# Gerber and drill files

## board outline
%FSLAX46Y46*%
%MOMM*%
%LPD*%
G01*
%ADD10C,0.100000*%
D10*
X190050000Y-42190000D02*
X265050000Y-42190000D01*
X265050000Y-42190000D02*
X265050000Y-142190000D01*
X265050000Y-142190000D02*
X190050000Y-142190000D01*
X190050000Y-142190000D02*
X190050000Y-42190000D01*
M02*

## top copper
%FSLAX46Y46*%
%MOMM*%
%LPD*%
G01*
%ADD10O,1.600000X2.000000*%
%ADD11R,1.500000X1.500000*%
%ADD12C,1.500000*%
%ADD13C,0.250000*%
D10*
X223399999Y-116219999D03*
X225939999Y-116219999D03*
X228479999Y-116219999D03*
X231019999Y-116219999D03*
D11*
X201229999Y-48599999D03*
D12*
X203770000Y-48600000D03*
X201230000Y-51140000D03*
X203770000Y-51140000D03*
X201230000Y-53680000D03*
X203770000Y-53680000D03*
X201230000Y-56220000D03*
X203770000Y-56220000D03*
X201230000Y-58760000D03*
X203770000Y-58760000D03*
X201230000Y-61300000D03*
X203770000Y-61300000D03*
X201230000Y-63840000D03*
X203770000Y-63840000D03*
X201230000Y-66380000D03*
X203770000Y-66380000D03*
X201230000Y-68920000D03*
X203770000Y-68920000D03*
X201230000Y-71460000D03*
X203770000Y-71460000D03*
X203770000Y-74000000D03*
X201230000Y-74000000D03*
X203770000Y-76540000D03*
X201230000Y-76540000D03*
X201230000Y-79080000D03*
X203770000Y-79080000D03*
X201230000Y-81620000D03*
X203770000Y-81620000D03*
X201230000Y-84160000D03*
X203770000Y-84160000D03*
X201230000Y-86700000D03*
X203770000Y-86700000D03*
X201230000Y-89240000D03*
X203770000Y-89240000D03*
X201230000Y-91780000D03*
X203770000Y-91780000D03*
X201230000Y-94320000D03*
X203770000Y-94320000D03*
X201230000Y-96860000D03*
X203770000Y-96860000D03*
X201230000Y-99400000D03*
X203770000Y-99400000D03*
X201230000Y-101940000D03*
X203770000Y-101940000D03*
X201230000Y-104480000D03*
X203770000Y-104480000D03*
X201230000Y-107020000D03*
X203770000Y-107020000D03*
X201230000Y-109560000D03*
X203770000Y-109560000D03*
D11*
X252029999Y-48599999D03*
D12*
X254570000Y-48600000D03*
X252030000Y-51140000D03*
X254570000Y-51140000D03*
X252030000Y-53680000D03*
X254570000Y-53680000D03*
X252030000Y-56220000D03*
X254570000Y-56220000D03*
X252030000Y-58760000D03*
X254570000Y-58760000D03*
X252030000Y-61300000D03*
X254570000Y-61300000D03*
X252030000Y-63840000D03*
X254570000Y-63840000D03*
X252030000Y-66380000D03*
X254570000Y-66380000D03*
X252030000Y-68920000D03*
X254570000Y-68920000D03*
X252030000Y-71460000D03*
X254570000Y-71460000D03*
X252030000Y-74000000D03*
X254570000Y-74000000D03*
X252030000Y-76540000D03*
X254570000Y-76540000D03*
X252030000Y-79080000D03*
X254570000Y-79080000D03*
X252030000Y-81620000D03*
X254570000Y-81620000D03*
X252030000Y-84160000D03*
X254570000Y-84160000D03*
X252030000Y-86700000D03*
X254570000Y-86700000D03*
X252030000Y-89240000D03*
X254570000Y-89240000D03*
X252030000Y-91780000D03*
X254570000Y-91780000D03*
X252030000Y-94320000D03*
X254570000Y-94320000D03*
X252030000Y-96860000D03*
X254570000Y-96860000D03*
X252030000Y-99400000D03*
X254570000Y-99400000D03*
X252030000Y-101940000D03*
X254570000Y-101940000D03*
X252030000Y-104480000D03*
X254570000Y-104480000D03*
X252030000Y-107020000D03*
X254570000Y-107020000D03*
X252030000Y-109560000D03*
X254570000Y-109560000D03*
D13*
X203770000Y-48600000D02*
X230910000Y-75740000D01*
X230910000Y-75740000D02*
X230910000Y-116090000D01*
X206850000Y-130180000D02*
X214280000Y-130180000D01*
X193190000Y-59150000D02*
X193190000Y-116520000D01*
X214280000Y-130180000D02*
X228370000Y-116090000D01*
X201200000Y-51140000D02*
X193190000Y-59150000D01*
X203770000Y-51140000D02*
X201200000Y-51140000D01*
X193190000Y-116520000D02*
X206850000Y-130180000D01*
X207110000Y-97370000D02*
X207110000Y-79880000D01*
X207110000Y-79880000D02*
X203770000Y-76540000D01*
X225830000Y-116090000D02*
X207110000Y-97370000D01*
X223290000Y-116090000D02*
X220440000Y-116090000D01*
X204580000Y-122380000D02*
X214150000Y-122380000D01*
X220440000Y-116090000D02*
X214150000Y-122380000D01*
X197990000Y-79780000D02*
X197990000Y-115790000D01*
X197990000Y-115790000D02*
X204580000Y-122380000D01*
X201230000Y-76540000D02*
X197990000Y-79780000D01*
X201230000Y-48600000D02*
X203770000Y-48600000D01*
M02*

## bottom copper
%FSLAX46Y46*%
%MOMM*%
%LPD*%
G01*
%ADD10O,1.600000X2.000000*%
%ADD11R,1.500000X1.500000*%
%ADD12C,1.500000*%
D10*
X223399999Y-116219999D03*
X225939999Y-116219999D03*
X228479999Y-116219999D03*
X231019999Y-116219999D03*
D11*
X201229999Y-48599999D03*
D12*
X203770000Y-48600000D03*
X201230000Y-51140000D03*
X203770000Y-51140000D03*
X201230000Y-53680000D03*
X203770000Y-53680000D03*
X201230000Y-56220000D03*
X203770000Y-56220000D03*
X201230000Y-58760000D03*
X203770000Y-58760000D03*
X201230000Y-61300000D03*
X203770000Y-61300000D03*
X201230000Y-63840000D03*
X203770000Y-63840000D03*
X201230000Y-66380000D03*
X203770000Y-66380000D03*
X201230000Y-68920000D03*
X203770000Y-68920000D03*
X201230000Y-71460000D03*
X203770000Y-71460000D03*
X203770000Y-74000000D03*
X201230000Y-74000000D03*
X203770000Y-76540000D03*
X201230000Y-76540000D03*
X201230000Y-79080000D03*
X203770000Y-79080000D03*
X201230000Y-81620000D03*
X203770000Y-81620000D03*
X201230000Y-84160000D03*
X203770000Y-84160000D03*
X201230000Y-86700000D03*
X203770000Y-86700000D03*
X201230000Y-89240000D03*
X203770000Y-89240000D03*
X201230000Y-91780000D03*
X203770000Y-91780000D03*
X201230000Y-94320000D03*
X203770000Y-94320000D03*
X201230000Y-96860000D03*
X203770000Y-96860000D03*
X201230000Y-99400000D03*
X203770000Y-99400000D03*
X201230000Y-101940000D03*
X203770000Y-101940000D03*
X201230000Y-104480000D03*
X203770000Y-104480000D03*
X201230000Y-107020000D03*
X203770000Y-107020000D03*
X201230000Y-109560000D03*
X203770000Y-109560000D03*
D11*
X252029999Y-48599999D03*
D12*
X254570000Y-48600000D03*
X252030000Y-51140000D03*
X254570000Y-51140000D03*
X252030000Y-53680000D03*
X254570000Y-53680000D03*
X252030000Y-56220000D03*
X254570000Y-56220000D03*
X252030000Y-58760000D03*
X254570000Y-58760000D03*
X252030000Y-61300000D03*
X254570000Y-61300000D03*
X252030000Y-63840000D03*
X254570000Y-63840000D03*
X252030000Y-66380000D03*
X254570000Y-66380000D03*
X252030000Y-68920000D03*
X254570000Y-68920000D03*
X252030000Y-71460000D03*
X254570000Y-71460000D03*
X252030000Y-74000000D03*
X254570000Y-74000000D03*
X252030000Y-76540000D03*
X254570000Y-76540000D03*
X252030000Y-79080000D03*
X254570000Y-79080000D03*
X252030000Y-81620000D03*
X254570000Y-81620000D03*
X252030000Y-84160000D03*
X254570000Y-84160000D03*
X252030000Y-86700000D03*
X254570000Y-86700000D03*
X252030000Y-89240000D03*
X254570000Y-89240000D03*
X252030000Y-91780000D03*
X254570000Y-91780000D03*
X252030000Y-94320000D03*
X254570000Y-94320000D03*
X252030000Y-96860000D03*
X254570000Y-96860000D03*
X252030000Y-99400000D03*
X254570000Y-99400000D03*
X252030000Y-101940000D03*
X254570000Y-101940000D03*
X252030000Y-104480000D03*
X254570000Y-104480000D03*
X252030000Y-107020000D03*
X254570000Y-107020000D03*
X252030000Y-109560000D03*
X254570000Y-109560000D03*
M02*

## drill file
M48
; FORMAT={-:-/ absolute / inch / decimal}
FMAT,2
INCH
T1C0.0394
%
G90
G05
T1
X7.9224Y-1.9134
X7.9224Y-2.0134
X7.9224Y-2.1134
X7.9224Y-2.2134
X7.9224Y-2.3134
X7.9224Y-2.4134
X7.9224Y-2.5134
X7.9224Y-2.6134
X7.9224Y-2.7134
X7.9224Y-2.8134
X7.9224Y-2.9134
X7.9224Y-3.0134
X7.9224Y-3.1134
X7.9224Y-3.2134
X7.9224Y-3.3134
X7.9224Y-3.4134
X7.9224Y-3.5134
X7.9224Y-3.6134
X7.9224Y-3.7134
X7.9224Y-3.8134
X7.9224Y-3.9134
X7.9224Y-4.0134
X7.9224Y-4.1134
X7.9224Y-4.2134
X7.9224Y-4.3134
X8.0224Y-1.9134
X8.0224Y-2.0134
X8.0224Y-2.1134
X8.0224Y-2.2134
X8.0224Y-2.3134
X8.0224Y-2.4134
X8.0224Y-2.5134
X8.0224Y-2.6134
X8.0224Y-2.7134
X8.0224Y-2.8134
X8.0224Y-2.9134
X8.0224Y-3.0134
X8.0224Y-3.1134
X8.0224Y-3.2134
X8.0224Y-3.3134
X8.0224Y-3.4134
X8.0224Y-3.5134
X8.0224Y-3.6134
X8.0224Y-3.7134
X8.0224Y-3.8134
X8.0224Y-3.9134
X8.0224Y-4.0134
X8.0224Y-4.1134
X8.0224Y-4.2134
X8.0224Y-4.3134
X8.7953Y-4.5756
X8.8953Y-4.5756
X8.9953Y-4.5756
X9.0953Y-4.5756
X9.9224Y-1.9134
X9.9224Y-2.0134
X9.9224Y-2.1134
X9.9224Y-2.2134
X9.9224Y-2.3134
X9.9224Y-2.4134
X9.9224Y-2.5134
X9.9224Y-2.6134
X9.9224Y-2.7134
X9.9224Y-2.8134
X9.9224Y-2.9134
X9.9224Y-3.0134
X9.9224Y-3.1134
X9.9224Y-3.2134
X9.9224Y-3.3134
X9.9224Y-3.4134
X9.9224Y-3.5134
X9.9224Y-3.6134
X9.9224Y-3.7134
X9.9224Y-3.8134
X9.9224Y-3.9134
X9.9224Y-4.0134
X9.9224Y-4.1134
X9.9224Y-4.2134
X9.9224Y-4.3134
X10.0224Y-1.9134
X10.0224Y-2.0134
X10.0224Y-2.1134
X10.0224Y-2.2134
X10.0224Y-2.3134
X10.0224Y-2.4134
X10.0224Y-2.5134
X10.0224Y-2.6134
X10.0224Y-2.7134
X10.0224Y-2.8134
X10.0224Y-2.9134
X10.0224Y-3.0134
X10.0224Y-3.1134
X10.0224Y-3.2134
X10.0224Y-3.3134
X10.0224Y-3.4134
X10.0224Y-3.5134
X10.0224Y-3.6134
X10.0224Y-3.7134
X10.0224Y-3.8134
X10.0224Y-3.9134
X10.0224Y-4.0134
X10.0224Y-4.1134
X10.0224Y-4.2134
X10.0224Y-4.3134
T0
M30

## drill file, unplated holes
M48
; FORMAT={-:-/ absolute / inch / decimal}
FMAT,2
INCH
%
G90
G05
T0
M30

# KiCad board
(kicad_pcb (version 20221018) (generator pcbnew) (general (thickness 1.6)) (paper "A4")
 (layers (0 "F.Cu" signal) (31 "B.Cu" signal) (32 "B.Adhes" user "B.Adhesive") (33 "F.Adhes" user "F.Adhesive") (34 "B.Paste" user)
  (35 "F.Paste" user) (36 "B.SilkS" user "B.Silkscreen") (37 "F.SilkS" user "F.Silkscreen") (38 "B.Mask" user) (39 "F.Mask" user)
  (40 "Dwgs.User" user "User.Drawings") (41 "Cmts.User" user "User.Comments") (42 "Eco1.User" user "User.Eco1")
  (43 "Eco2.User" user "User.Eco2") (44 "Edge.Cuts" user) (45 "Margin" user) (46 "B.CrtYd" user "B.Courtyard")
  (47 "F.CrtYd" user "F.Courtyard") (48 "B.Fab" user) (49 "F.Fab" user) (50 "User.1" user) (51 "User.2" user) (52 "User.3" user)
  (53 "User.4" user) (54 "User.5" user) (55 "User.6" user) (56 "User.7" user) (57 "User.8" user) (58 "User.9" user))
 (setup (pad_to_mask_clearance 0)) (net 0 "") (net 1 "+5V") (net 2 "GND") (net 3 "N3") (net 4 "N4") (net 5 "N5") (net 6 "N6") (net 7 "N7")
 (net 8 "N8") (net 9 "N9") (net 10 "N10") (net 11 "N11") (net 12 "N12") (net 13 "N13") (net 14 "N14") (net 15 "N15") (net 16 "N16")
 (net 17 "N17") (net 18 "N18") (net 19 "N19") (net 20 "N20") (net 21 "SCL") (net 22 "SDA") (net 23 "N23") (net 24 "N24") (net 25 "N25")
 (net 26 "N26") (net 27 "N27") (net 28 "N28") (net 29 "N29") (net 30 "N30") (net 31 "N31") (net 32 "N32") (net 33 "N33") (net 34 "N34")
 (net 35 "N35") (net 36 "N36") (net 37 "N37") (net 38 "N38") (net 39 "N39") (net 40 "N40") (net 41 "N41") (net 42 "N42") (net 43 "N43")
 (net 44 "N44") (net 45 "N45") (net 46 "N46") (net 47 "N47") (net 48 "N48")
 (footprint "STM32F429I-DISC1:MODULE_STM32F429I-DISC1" (layer "F.Cu") (at 227.9 74.43)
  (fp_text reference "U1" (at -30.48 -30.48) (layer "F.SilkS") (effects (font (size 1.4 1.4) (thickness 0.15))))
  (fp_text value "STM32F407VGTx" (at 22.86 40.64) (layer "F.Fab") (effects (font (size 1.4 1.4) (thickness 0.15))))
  (pad "P1_1" thru_hole rect (at -26.67 -25.83) (size 1.5 1.5) (drill 1) (layers "*.Cu" "*.Mask") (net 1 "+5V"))
  (pad "P1_2" thru_hole circle (at -24.13 -25.83) (size 1.5 1.5) (drill 1) (layers "*.Cu" "*.Mask") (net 1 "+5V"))
  (pad "P1_3" thru_hole circle (at -26.67 -23.29) (size 1.5 1.5) (drill 1) (layers "*.Cu" "*.Mask") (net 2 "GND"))
  (pad "P1_4" thru_hole circle (at -24.13 -23.29) (size 1.5 1.5) (drill 1) (layers "*.Cu" "*.Mask") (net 2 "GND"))
  (pad "P1_5" thru_hole circle (at -26.67 -20.75) (size 1.5 1.5) (drill 1) (layers "*.Cu" "*.Mask") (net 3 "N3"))
  (pad "P1_6" thru_hole circle (at -24.13 -20.75) (size 1.5 1.5) (drill 1) (layers "*.Cu" "*.Mask") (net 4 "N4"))
  (pad "P1_7" thru_hole circle (at -26.67 -18.21) (size 1.5 1.5) (drill 1) (layers "*.Cu" "*.Mask") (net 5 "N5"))
  (pad "P1_8" thru_hole circle (at -24.13 -18.21) (size 1.5 1.5) (drill 1) (layers "*.Cu" "*.Mask") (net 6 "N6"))
  (pad "P1_9" thru_hole circle (at -26.67 -15.67) (size 1.5 1.5) (drill 1) (layers "*.Cu" "*.Mask") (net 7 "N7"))
  (pad "P1_10" thru_hole circle (at -24.13 -15.67) (size 1.5 1.5) (drill 1) (layers "*.Cu" "*.Mask") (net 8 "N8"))
  (pad "P1_11" thru_hole circle (at -26.67 -13.13) (size 1.5 1.5) (drill 1) (layers "*.Cu" "*.Mask") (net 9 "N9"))
  (pad "P1_12" thru_hole circle (at -24.13 -13.13) (size 1.5 1.5) (drill 1) (layers "*.Cu" "*.Mask") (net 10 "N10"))
  (pad "P1_13" thru_hole circle (at -26.67 -10.59) (size 1.5 1.5) (drill 1) (layers "*.Cu" "*.Mask") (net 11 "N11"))
  (pad "P1_14" thru_hole circle (at -24.13 -10.59) (size 1.5 1.5) (drill 1) (layers "*.Cu" "*.Mask") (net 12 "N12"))
  (pad "P1_15" thru_hole circle (at -26.67 -8.05) (size 1.5 1.5) (drill 1) (layers "*.Cu" "*.Mask") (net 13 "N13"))
  (pad "P1_16" thru_hole circle (at -24.13 -8.05) (size 1.5 1.5) (drill 1) (layers "*.Cu" "*.Mask") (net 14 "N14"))
  (pad "P1_17" thru_hole circle (at -26.67 -5.51) (size 1.5 1.5) (drill 1) (layers "*.Cu" "*.Mask") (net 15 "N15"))
  (pad "P1_18" thru_hole circle (at -24.13 -5.51) (size 1.5 1.5) (drill 1) (layers "*.Cu" "*.Mask") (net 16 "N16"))
  (pad "P1_19" thru_hole circle (at -26.67 -2.97) (size 1.5 1.5) (drill 1) (layers "*.Cu" "*.Mask") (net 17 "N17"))
  (pad "P1_20" thru_hole circle (at -24.13 -2.97) (size 1.5 1.5) (drill 1) (layers "*.Cu" "*.Mask") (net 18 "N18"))
  (pad "P1_21" thru_hole circle (at -24.13 -0.43) (size 1.5 1.5) (drill 1) (layers "*.Cu" "*.Mask") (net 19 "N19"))
  (pad "P1_22" thru_hole circle (at -26.67 -0.43) (size 1.5 1.5) (drill 1) (layers "*.Cu" "*.Mask") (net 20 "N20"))
  (pad "P1_23" thru_hole circle (at -24.13 2.11) (size 1.5 1.5) (drill 1) (layers "*.Cu" "*.Mask") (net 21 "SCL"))
  (pad "P1_24" thru_hole circle (at -26.67 2.11) (size 1.5 1.5) (drill 1) (layers "*.Cu" "*.Mask") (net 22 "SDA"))
  (pad "P1_25" thru_hole circle (at -26.67 4.65) (size 1.5 1.5) (drill 1) (layers "*.Cu" "*.Mask") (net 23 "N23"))
  (pad "P1_26" thru_hole circle (at -24.13 4.65) (size 1.5 1.5) (drill 1) (layers "*.Cu" "*.Mask") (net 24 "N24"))
  (pad "P1_27" thru_hole circle (at -26.67 7.19) (size 1.5 1.5) (drill 1) (layers "*.Cu" "*.Mask") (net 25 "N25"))
  (pad "P1_28" thru_hole circle (at -24.13 7.19) (size 1.5 1.5) (drill 1) (layers "*.Cu" "*.Mask") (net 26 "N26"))
  (pad "P1_29" thru_hole circle (at -26.67 9.73) (size 1.5 1.5) (drill 1) (layers "*.Cu" "*.Mask") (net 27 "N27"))
  (pad "P1_30" thru_hole circle (at -24.13 9.73) (size 1.5 1.5) (drill 1) (layers "*.Cu" "*.Mask") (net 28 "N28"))
  (pad "P1_31" thru_hole circle (at -26.67 12.27) (size 1.5 1.5) (drill 1) (layers "*.Cu" "*.Mask") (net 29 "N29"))
  (pad "P1_32" thru_hole circle (at -24.13 12.27) (size 1.5 1.5) (drill 1) (layers "*.Cu" "*.Mask") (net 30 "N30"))
  (pad "P1_33" thru_hole circle (at -26.67 14.81) (size 1.5 1.5) (drill 1) (layers "*.Cu" "*.Mask") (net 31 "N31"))
  (pad "P1_34" thru_hole circle (at -24.13 14.81) (size 1.5 1.5) (drill 1) (layers "*.Cu" "*.Mask") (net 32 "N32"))
  (pad "P1_35" thru_hole circle (at -26.67 17.35) (size 1.5 1.5) (drill 1) (layers "*.Cu" "*.Mask") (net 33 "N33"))
  (pad "P1_36" thru_hole circle (at -24.13 17.35) (size 1.5 1.5) (drill 1) (layers "*.Cu" "*.Mask") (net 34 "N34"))
  (pad "P1_37" thru_hole circle (at -26.67 19.89) (size 1.5 1.5) (drill 1) (layers "*.Cu" "*.Mask") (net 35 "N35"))
  (pad "P1_38" thru_hole circle (at -24.13 19.89) (size 1.5 1.5) (drill 1) (layers "*.Cu" "*.Mask") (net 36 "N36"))
  (pad "P1_39" thru_hole circle (at -26.67 22.43) (size 1.5 1.5) (drill 1) (layers "*.Cu" "*.Mask") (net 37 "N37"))
  (pad "P1_40" thru_hole circle (at -24.13 22.43) (size 1.5 1.5) (drill 1) (layers "*.Cu" "*.Mask") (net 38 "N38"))
  (pad "P1_41" thru_hole circle (at -26.67 24.97) (size 1.5 1.5) (drill 1) (layers "*.Cu" "*.Mask") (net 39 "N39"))
  (pad "P1_42" thru_hole circle (at -24.13 24.97) (size 1.5 1.5) (drill 1) (layers "*.Cu" "*.Mask") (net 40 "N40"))
  (pad "P1_43" thru_hole circle (at -26.67 27.51) (size 1.5 1.5) (drill 1) (layers "*.Cu" "*.Mask") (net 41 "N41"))
  (pad "P1_44" thru_hole circle (at -24.13 27.51) (size 1.5 1.5) (drill 1) (layers "*.Cu" "*.Mask") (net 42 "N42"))
  (pad "P1_45" thru_hole circle (at -26.67 30.05) (size 1.5 1.5) (drill 1) (layers "*.Cu" "*.Mask") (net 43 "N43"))
  (pad "P1_46" thru_hole circle (at -24.13 30.05) (size 1.5 1.5) (drill 1) (layers "*.Cu" "*.Mask") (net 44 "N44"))
  (pad "P1_47" thru_hole circle (at -26.67 32.59) (size 1.5 1.5) (drill 1) (layers "*.Cu" "*.Mask") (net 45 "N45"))
  (pad "P1_48" thru_hole circle (at -24.13 32.59) (size 1.5 1.5) (drill 1) (layers "*.Cu" "*.Mask") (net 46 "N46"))
  (pad "P1_49" thru_hole circle (at -26.67 35.13) (size 1.5 1.5) (drill 1) (layers "*.Cu" "*.Mask") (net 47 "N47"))
  (pad "P1_50" thru_hole circle (at -24.13 35.13) (size 1.5 1.5) (drill 1) (layers "*.Cu" "*.Mask") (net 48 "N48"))
  (pad "P2_1" thru_hole rect (at 24.13 -25.83) (size 1.5 1.5) (drill 1) (layers "*.Cu" "*.Mask"))
  (pad "P2_2" thru_hole circle (at 26.67 -25.83) (size 1.5 1.5) (drill 1) (layers "*.Cu" "*.Mask"))
  (pad "P2_3" thru_hole circle (at 24.13 -23.29) (size 1.5 1.5) (drill 1) (layers "*.Cu" "*.Mask"))
  (pad "P2_4" thru_hole circle (at 26.67 -23.29) (size 1.5 1.5) (drill 1) (layers "*.Cu" "*.Mask"))
  (pad "P2_5" thru_hole circle (at 24.13 -20.75) (size 1.5 1.5) (drill 1) (layers "*.Cu" "*.Mask"))
  (pad "P2_6" thru_hole circle (at 26.67 -20.75) (size 1.5 1.5) (drill 1) (layers "*.Cu" "*.Mask"))
  (pad "P2_7" thru_hole circle (at 24.13 -18.21) (size 1.5 1.5) (drill 1) (layers "*.Cu" "*.Mask"))
  (pad "P2_8" thru_hole circle (at 26.67 -18.21) (size 1.5 1.5) (drill 1) (layers "*.Cu" "*.Mask"))
  (pad "P2_9" thru_hole circle (at 24.13 -15.67) (size 1.5 1.5) (drill 1) (layers "*.Cu" "*.Mask"))
  (pad "P2_10" thru_hole circle (at 26.67 -15.67) (size 1.5 1.5) (drill 1) (layers "*.Cu" "*.Mask"))
  (pad "P2_11" thru_hole circle (at 24.13 -13.13) (size 1.5 1.5) (drill 1) (layers "*.Cu" "*.Mask"))
  (pad "P2_12" thru_hole circle (at 26.67 -13.13) (size 1.5 1.5) (drill 1) (layers "*.Cu" "*.Mask"))
  (pad "P2_13" thru_hole circle (at 24.13 -10.59) (size 1.5 1.5) (drill 1) (layers "*.Cu" "*.Mask"))
  (pad "P2_14" thru_hole circle (at 26.67 -10.59) (size 1.5 1.5) (drill 1) (layers "*.Cu" "*.Mask"))
  (pad "P2_15" thru_hole circle (at 24.13 -8.05) (size 1.5 1.5) (drill 1) (layers "*.Cu" "*.Mask"))
  (pad "P2_16" thru_hole circle (at 26.67 -8.05) (size 1.5 1.5) (drill 1) (layers "*.Cu" "*.Mask"))
  (pad "P2_17" thru_hole circle (at 24.13 -5.51) (size 1.5 1.5) (drill 1) (layers "*.Cu" "*.Mask"))
  (pad "P2_18" thru_hole circle (at 26.67 -5.51) (size 1.5 1.5) (drill 1) (layers "*.Cu" "*.Mask"))
  (pad "P2_19" thru_hole circle (at 24.13 -2.97) (size 1.5 1.5) (drill 1) (layers "*.Cu" "*.Mask"))
  (pad "P2_20" thru_hole circle (at 26.67 -2.97) (size 1.5 1.5) (drill 1) (layers "*.Cu" "*.Mask"))
  (pad "P2_21" thru_hole circle (at 24.13 -0.43) (size 1.5 1.5) (drill 1) (layers "*.Cu" "*.Mask"))
  (pad "P2_22" thru_hole circle (at 26.67 -0.43) (size 1.5 1.5) (drill 1) (layers "*.Cu" "*.Mask"))
  (pad "P2_23" thru_hole circle (at 24.13 2.11) (size 1.5 1.5) (drill 1) (layers "*.Cu" "*.Mask"))
  (pad "P2_24" thru_hole circle (at 26.67 2.11) (size 1.5 1.5) (drill 1) (layers "*.Cu" "*.Mask"))
  (pad "P2_25" thru_hole circle (at 24.13 4.65) (size 1.5 1.5) (drill 1) (layers "*.Cu" "*.Mask"))
  (pad "P2_26" thru_hole circle (at 26.67 4.65) (size 1.5 1.5) (drill 1) (layers "*.Cu" "*.Mask"))
  (pad "P2_27" thru_hole circle (at 24.13 7.19) (size 1.5 1.5) (drill 1) (layers "*.Cu" "*.Mask"))
  (pad "P2_28" thru_hole circle (at 26.67 7.19) (size 1.5 1.5) (drill 1) (layers "*.Cu" "*.Mask"))
  (pad "P2_29" thru_hole circle (at 24.13 9.73) (size 1.5 1.5) (drill 1) (layers "*.Cu" "*.Mask"))
  (pad "P2_30" thru_hole circle (at 26.67 9.73) (size 1.5 1.5) (drill 1) (layers "*.Cu" "*.Mask"))
  (pad "P2_31" thru_hole circle (at 24.13 12.27) (size 1.5 1.5) (drill 1) (layers "*.Cu" "*.Mask"))
  (pad "P2_32" thru_hole circle (at 26.67 12.27) (size 1.5 1.5) (drill 1) (layers "*.Cu" "*.Mask"))
  (pad "P2_33" thru_hole circle (at 24.13 14.81) (size 1.5 1.5) (drill 1) (layers "*.Cu" "*.Mask"))
  (pad "P2_34" thru_hole circle (at 26.67 14.81) (size 1.5 1.5) (drill 1) (layers "*.Cu" "*.Mask"))
  (pad "P2_35" thru_hole circle (at 24.13 17.35) (size 1.5 1.5) (drill 1) (layers "*.Cu" "*.Mask"))
  (pad "P2_36" thru_hole circle (at 26.67 17.35) (size 1.5 1.5) (drill 1) (layers "*.Cu" "*.Mask"))
  (pad "P2_37" thru_hole circle (at 24.13 19.89) (size 1.5 1.5) (drill 1) (layers "*.Cu" "*.Mask"))
  (pad "P2_38" thru_hole circle (at 26.67 19.89) (size 1.5 1.5) (drill 1) (layers "*.Cu" "*.Mask"))
  (pad "P2_39" thru_hole circle (at 24.13 22.43) (size 1.5 1.5) (drill 1) (layers "*.Cu" "*.Mask"))
  (pad "P2_40" thru_hole circle (at 26.67 22.43) (size 1.5 1.5) (drill 1) (layers "*.Cu" "*.Mask"))
  (pad "P2_41" thru_hole circle (at 24.13 24.97) (size 1.5 1.5) (drill 1) (layers "*.Cu" "*.Mask"))
  (pad "P2_42" thru_hole circle (at 26.67 24.97) (size 1.5 1.5) (drill 1) (layers "*.Cu" "*.Mask"))
  (pad "P2_43" thru_hole circle (at 24.13 27.51) (size 1.5 1.5) (drill 1) (layers "*.Cu" "*.Mask"))
  (pad "P2_44" thru_hole circle (at 26.67 27.51) (size 1.5 1.5) (drill 1) (layers "*.Cu" "*.Mask"))
  (pad "P2_45" thru_hole circle (at 24.13 30.05) (size 1.5 1.5) (drill 1) (layers "*.Cu" "*.Mask"))
  (pad "P2_46" thru_hole circle (at 26.67 30.05) (size 1.5 1.5) (drill 1) (layers "*.Cu" "*.Mask"))
  (pad "P2_47" thru_hole circle (at 24.13 32.59) (size 1.5 1.5) (drill 1) (layers "*.Cu" "*.Mask"))
  (pad "P2_48" thru_hole circle (at 26.67 32.59) (size 1.5 1.5) (drill 1) (layers "*.Cu" "*.Mask"))
  (pad "P2_49" thru_hole circle (at 24.13 35.13) (size 1.5 1.5) (drill 1) (layers "*.Cu" "*.Mask"))
  (pad "P2_50" thru_hole circle (at 26.67 35.13) (size 1.5 1.5) (drill 1) (layers "*.Cu" "*.Mask")))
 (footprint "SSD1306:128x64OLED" (layer "B.Cu") (at 227.4 126.82 180)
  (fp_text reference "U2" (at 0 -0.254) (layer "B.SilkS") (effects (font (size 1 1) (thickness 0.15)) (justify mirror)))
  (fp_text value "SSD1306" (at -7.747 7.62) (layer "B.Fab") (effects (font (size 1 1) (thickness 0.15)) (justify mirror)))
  (pad "1" thru_hole oval (at -3.62 10.6 90) (size 2 1.6) (drill 1) (layers "*.Cu" "*.Mask") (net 1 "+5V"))
  (pad "2" thru_hole oval (at -1.08 10.6 90) (size 2 1.6) (drill 1) (layers "*.Cu" "*.Mask") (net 2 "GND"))
  (pad "3" thru_hole oval (at 1.46 10.6 90) (size 2 1.6) (drill 1) (layers "*.Cu" "*.Mask") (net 21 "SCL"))
  (pad "4" thru_hole oval (at 4 10.6 90) (size 2 1.6) (drill 1) (layers "*.Cu" "*.Mask") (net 22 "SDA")))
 (gr_rect (start 190.05 42.19) (end 265.05 142.19) (stroke (width 0.1) (type default)) (fill none) (layer "Edge.Cuts"))
 (segment (start 207.11 79.88) (end 203.77 76.54) (width 0.25) (layer "F.Cu") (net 21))
 (segment (start 207.11 97.37) (end 207.11 79.88) (width 0.25) (layer "F.Cu") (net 21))
 (segment (start 225.83 116.09) (end 207.11 97.37) (width 0.25) (layer "F.Cu") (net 21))
 (segment (start 197.99 79.78) (end 197.99 115.79) (width 0.25) (layer "F.Cu") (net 22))
 (segment (start 204.58 122.38) (end 214.15 122.38) (width 0.25) (layer "F.Cu") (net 22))
 (segment (start 220.44 116.09) (end 214.15 122.38) (width 0.25) (layer "F.Cu") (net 22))
 (segment (start 197.99 115.79) (end 204.58 122.38) (width 0.25) (layer "F.Cu") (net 22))
 (segment (start 223.29 116.09) (end 220.44 116.09) (width 0.25) (layer "F.Cu") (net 22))
 (segment (start 201.23 76.54) (end 197.99 79.78) (width 0.25) (layer "F.Cu") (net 22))
 (segment (start 206.85 130.18) (end 214.28 130.18) (width 0.25) (layer "F.Cu") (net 2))
 (segment (start 203.77 51.14) (end 201.2 51.14) (width 0.25) (layer "F.Cu") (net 2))
 (segment (start 201.2 51.14) (end 193.19 59.15) (width 0.25) (layer "F.Cu") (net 2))
 (segment (start 214.28 130.18) (end 228.37 116.09) (width 0.25) (layer "F.Cu") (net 2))
 (segment (start 193.19 116.52) (end 206.85 130.18) (width 0.25) (layer "F.Cu") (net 2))
 (segment (start 193.19 59.15) (end 193.19 116.52) (width 0.25) (layer "F.Cu") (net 2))
 (segment (start 230.91 75.74) (end 230.91 116.09) (width 0.25) (layer "F.Cu") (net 1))
 (segment (start 201.23 48.6) (end 203.77 48.6) (width 0.25) (layer "F.Cu") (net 1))
 (segment (start 203.77 48.6) (end 230.91 75.74) (width 0.25) (layer "F.Cu") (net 1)))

